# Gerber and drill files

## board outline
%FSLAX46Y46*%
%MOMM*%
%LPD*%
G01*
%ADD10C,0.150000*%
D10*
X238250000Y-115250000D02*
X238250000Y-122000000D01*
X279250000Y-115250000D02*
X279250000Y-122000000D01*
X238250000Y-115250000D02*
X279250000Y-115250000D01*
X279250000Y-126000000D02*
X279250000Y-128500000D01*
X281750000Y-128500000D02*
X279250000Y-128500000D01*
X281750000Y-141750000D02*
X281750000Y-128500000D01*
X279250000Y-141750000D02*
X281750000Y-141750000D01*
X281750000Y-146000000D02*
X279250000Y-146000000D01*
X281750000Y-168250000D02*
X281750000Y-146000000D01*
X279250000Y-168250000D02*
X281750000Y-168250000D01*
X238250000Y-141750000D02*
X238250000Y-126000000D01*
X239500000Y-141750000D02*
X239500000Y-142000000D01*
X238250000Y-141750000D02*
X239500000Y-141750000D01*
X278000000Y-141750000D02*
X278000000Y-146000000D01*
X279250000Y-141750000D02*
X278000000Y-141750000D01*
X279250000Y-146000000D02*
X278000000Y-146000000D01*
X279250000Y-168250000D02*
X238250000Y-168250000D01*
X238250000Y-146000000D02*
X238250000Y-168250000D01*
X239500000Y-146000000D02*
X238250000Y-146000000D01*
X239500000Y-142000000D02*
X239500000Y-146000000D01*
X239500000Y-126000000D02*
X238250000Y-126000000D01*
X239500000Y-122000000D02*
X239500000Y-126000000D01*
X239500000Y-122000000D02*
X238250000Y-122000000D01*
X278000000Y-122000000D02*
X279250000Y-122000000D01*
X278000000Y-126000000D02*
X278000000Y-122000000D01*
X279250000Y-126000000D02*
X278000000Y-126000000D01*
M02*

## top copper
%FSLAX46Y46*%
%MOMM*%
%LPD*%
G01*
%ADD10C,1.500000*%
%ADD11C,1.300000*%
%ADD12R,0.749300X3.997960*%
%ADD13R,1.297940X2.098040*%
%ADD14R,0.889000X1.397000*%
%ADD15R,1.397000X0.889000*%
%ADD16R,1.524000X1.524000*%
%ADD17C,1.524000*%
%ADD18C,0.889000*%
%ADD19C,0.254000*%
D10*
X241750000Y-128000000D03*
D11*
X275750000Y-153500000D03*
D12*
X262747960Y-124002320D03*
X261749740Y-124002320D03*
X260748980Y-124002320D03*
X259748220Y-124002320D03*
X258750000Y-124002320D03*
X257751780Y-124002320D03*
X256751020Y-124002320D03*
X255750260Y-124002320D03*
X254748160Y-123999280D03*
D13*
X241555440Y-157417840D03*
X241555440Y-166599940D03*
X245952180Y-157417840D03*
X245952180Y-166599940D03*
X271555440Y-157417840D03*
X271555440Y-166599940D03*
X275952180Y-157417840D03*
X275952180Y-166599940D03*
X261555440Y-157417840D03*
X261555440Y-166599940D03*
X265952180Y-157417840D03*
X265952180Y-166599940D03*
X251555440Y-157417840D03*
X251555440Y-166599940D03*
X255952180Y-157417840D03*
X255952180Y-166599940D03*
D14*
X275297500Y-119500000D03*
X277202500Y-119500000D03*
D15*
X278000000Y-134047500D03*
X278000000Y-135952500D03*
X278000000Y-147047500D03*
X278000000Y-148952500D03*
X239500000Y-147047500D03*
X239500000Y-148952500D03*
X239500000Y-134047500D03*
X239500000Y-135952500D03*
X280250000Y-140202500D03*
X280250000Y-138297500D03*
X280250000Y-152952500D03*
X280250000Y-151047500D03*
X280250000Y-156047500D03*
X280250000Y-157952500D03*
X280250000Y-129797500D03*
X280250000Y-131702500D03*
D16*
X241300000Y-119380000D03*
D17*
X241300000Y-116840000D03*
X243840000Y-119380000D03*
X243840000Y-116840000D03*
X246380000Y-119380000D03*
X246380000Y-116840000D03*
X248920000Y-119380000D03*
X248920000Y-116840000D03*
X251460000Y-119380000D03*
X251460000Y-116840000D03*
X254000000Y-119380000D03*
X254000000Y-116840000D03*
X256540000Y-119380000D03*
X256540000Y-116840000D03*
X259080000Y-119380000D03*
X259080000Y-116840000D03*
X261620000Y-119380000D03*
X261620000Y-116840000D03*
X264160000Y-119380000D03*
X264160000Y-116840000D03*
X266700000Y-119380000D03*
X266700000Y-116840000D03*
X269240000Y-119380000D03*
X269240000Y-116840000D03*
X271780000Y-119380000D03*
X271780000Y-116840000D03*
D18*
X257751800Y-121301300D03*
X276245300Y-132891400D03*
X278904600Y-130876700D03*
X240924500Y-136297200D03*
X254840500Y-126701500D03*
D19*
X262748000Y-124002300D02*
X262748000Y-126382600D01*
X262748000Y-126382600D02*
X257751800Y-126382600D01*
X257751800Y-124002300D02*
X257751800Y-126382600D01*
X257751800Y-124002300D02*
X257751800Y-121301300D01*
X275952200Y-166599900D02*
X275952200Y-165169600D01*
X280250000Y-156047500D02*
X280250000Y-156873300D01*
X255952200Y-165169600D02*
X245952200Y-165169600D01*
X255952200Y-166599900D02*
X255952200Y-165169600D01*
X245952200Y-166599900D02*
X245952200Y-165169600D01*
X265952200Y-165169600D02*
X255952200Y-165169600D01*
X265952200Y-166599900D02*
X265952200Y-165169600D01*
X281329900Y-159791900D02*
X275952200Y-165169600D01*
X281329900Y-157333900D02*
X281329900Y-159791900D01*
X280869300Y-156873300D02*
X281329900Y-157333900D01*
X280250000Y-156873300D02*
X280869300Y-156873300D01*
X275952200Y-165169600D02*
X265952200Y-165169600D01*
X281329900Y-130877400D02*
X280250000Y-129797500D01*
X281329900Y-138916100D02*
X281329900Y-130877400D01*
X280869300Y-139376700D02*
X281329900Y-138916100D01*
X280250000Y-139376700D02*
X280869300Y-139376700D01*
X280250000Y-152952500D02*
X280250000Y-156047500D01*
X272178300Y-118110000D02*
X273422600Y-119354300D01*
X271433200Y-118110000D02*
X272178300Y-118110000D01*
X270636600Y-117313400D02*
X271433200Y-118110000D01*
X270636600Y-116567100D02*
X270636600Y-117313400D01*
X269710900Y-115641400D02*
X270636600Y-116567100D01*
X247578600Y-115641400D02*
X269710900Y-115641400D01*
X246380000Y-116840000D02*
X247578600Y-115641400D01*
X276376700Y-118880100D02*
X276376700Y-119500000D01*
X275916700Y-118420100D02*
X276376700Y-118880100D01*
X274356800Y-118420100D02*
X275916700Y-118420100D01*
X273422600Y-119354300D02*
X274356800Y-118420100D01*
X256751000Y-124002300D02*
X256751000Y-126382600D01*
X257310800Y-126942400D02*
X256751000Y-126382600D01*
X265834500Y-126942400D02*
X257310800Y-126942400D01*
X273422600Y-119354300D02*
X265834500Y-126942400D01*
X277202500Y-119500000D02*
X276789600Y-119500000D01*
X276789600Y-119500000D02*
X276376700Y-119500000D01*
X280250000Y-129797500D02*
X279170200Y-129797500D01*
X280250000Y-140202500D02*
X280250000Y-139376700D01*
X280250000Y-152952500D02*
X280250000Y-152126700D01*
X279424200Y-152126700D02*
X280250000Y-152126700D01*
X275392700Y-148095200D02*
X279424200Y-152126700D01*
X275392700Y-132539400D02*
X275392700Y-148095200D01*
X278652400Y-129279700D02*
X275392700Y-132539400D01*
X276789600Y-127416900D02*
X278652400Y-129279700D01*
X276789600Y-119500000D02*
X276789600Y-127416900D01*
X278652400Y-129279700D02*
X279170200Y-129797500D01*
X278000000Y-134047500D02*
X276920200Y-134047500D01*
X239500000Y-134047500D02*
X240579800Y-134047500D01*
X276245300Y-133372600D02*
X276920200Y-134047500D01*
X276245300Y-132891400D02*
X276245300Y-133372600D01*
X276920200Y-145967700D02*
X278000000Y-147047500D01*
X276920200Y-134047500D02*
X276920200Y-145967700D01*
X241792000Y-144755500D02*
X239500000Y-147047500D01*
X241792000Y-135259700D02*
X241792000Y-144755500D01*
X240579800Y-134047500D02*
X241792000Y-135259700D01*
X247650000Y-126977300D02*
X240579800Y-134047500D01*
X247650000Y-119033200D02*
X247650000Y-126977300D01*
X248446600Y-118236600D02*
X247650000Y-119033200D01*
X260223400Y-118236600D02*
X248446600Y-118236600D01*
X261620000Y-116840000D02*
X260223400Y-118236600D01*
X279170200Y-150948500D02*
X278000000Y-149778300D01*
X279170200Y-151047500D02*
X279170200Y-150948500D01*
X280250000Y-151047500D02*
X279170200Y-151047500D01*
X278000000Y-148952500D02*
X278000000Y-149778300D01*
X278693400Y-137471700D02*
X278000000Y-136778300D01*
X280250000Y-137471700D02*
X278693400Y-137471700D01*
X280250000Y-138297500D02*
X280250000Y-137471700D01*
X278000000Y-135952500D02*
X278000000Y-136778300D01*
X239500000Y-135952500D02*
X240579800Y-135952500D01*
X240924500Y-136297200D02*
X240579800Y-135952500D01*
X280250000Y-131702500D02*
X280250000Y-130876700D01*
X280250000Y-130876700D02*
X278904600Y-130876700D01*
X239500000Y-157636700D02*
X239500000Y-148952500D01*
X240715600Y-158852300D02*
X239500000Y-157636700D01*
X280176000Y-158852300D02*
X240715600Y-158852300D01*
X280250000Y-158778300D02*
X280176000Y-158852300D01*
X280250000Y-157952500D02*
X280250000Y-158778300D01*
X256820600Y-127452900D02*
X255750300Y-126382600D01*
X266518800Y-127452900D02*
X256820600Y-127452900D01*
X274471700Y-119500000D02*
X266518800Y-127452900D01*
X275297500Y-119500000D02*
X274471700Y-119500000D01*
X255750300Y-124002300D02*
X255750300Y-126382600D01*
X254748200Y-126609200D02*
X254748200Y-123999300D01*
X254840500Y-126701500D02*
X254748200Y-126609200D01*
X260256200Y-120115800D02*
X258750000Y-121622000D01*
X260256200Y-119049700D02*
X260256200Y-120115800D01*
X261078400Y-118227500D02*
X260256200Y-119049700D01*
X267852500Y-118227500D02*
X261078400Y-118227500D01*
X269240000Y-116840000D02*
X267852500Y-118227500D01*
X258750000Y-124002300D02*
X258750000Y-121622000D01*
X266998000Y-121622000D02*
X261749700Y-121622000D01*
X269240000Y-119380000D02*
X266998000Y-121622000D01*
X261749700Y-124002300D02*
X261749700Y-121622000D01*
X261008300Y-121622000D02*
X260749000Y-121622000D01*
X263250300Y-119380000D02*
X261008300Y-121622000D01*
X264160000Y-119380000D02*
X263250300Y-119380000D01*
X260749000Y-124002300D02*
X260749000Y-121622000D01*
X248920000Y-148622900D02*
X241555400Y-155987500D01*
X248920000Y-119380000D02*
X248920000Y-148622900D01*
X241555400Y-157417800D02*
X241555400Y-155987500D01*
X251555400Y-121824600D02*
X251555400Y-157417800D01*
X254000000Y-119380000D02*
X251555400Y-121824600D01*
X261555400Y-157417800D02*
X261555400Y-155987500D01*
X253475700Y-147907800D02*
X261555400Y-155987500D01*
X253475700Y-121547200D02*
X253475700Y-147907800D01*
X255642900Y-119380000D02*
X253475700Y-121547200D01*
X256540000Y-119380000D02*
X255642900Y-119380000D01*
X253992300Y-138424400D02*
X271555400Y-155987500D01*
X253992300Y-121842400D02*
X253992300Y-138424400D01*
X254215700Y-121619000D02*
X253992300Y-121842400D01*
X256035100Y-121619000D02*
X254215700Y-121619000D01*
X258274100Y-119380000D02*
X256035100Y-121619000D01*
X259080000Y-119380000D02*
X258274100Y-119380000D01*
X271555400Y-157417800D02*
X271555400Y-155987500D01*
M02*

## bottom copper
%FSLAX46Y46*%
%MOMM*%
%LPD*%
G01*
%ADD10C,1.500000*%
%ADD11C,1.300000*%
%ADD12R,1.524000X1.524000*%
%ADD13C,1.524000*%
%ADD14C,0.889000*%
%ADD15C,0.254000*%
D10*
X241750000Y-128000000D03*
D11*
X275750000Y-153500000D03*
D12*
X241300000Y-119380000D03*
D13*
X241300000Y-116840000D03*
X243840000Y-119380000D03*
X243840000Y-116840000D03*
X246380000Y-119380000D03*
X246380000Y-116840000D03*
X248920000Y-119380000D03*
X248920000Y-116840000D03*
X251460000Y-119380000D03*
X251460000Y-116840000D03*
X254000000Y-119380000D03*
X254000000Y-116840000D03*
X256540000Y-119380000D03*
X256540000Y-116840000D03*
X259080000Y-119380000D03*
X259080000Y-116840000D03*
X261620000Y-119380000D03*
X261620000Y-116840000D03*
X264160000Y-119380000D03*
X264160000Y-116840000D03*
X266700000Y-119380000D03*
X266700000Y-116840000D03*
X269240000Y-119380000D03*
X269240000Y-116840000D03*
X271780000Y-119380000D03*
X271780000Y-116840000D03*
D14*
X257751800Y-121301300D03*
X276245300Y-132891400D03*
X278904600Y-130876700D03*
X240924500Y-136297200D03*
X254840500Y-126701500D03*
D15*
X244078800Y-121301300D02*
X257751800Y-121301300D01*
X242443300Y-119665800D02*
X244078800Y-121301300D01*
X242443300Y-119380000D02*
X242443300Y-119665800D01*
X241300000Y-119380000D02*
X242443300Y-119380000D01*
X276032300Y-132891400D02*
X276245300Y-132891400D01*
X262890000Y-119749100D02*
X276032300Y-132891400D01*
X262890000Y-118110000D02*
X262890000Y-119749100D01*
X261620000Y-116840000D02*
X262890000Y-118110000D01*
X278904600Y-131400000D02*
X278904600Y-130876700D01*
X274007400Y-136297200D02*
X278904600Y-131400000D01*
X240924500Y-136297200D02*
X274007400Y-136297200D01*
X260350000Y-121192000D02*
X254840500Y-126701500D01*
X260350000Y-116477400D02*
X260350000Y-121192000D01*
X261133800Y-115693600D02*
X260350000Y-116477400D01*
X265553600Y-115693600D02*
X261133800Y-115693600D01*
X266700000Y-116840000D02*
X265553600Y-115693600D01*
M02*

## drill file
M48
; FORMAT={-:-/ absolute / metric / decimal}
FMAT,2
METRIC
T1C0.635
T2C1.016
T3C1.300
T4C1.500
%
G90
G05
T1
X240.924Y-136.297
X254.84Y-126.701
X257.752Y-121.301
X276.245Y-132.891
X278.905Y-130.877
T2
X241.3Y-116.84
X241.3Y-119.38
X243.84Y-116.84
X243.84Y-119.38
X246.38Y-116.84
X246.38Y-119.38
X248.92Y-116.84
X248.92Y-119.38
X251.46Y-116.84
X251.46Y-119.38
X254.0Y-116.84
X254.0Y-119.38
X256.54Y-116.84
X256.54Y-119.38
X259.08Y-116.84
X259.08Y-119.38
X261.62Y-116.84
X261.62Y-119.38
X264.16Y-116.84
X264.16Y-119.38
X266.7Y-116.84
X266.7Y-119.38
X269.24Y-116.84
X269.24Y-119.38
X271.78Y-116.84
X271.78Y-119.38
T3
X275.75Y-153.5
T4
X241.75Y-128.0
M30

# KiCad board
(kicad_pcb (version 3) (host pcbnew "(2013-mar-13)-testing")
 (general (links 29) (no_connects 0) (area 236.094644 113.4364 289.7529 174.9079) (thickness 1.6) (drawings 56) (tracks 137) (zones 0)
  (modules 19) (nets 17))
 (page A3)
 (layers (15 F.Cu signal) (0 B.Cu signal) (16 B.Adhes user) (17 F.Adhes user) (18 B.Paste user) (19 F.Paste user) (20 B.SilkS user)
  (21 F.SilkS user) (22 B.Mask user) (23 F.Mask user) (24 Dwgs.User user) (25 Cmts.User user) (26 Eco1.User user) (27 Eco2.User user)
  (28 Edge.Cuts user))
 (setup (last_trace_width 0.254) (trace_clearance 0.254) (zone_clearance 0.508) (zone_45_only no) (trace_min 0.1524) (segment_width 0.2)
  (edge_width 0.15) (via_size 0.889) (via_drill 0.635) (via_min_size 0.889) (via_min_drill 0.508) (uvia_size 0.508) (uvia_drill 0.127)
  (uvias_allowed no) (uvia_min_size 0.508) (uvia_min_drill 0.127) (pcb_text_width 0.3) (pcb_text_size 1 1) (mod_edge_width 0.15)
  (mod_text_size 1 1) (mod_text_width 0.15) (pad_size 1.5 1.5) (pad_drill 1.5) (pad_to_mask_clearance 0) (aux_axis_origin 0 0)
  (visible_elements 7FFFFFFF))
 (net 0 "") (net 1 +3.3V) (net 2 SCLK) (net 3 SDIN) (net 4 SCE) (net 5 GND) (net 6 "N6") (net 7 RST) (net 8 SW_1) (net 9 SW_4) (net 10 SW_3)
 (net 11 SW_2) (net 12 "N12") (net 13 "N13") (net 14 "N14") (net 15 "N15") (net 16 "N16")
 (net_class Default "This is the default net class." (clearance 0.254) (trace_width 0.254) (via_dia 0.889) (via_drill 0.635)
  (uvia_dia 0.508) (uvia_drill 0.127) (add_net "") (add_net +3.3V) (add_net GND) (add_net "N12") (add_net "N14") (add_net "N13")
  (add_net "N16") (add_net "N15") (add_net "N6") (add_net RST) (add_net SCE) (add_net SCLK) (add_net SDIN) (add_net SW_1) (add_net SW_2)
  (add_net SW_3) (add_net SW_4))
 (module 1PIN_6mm (layer F.Cu) (at 241.75 128)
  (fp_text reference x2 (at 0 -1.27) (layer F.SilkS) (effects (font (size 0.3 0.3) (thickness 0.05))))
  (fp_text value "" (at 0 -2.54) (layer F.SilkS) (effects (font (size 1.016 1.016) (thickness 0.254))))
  (pad 1 thru_hole circle (at 0 0) (size 1.5 1.5) (drill 1.5) (layers *.Cu *.Mask F.SilkS)))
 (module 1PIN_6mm (layer F.Cu) (at 275.75 153.5)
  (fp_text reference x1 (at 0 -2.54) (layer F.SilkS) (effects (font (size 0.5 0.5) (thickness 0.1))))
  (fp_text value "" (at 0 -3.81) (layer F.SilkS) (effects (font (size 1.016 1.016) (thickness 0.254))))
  (pad 1 thru_hole circle (at 0 0) (size 1.3 1.3) (drill 1.3) (layers *.Cu *.Mask F.SilkS)))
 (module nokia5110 (layer F.Cu) (at 258.75 141)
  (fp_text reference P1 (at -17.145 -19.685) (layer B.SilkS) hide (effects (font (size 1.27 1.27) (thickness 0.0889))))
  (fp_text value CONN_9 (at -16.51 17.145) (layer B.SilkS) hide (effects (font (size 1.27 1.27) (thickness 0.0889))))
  (pad 9 smd rect (at 3.99796 -16.99768) (size 0.7493 3.99796) (layers F.Cu F.Paste F.Mask) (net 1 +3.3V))
  (pad 8 smd rect (at 2.99974 -16.99768) (size 0.7493 3.99796) (layers F.Cu F.Paste F.Mask) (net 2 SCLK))
  (pad 7 smd rect (at 1.99898 -16.99768) (size 0.7493 3.99796) (layers F.Cu F.Paste F.Mask) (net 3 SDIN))
  (pad 6 smd rect (at 0.99822 -16.99768) (size 0.7493 3.99796) (layers F.Cu F.Paste F.Mask))
  (pad 5 smd rect (at 0 -16.99768) (size 0.7493 3.99796) (layers F.Cu F.Paste F.Mask) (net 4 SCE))
  (pad 4 smd rect (at -0.99822 -16.99768) (size 0.7493 3.99796) (layers F.Cu F.Paste F.Mask) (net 1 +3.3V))
  (pad 3 smd rect (at -1.99898 -16.99768) (size 0.7493 3.99796) (layers F.Cu F.Paste F.Mask) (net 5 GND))
  (pad 2 smd rect (at -2.99974 -16.99768) (size 0.7493 3.99796) (layers F.Cu F.Paste F.Mask) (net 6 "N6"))
  (pad 1 smd rect (at -4.00184 -17.00072) (size 0.7493 3.99796) (layers F.Cu F.Paste F.Mask) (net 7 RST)))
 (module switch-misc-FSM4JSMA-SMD (layer F.Cu) (at 243.75 162)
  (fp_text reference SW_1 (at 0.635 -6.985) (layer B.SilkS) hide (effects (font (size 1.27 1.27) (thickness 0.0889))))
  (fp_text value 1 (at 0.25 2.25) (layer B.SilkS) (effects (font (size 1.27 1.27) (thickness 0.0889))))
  (pad P$1 smd rect (at -2.19456 -4.58216) (size 1.29794 2.09804) (layers F.Cu F.Paste F.Mask) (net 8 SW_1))
  (pad P$2 smd rect (at -2.19456 4.59994) (size 1.29794 2.09804) (layers F.Cu F.Paste F.Mask))
  (pad P$3 smd rect (at 2.20218 -4.58216) (size 1.29794 2.09804) (layers F.Cu F.Paste F.Mask))
  (pad P$4 smd rect (at 2.20218 4.59994) (size 1.29794 2.09804) (layers F.Cu F.Paste F.Mask) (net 5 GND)))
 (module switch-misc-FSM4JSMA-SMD (layer F.Cu) (at 273.75 162)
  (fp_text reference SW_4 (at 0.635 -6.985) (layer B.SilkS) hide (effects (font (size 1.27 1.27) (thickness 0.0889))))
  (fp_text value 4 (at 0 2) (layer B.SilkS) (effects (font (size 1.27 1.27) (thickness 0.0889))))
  (pad P$1 smd rect (at -2.19456 -4.58216) (size 1.29794 2.09804) (layers F.Cu F.Paste F.Mask) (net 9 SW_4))
  (pad P$2 smd rect (at -2.19456 4.59994) (size 1.29794 2.09804) (layers F.Cu F.Paste F.Mask))
  (pad P$3 smd rect (at 2.20218 -4.58216) (size 1.29794 2.09804) (layers F.Cu F.Paste F.Mask))
  (pad P$4 smd rect (at 2.20218 4.59994) (size 1.29794 2.09804) (layers F.Cu F.Paste F.Mask) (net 5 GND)))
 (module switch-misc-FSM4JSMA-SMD (layer F.Cu) (at 263.75 162)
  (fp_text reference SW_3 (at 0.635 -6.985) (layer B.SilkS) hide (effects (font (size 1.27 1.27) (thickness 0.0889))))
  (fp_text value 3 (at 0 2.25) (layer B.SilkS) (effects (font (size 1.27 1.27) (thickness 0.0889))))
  (pad P$1 smd rect (at -2.19456 -4.58216) (size 1.29794 2.09804) (layers F.Cu F.Paste F.Mask) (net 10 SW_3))
  (pad P$2 smd rect (at -2.19456 4.59994) (size 1.29794 2.09804) (layers F.Cu F.Paste F.Mask))
  (pad P$3 smd rect (at 2.20218 -4.58216) (size 1.29794 2.09804) (layers F.Cu F.Paste F.Mask))
  (pad P$4 smd rect (at 2.20218 4.59994) (size 1.29794 2.09804) (layers F.Cu F.Paste F.Mask) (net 5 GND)))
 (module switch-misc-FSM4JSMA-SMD (layer F.Cu) (at 253.75 162)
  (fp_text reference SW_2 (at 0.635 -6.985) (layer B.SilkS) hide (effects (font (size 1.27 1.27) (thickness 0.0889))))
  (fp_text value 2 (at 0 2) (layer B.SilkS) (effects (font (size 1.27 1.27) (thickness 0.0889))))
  (pad P$1 smd rect (at -2.19456 -4.58216) (size 1.29794 2.09804) (layers F.Cu F.Paste F.Mask) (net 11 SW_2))
  (pad P$2 smd rect (at -2.19456 4.59994) (size 1.29794 2.09804) (layers F.Cu F.Paste F.Mask))
  (pad P$3 smd rect (at 2.20218 -4.58216) (size 1.29794 2.09804) (layers F.Cu F.Paste F.Mask))
  (pad P$4 smd rect (at 2.20218 4.59994) (size 1.29794 2.09804) (layers F.Cu F.Paste F.Mask) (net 5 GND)))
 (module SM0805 (layer F.Cu) (at 276.25 119.5)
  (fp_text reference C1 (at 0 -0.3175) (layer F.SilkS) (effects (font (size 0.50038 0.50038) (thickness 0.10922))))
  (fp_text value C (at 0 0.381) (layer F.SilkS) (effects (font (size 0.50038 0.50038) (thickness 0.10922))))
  (pad 1 smd rect (at -0.9525 0) (size 0.889 1.397) (layers F.Cu F.Paste F.Mask) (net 6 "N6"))
  (pad 2 smd rect (at 0.9525 0) (size 0.889 1.397) (layers F.Cu F.Paste F.Mask) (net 5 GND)))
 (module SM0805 (layer F.Cu) (at 278 135 270)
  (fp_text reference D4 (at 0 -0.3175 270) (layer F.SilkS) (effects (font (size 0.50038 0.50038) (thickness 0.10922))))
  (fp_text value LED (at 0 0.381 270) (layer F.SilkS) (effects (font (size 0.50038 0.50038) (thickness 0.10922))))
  (pad 1 smd rect (at -0.9525 0 270) (size 0.889 1.397) (layers F.Cu F.Paste F.Mask) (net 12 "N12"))
  (pad 2 smd rect (at 0.9525 0 270) (size 0.889 1.397) (layers F.Cu F.Paste F.Mask) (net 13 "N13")))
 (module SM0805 (layer F.Cu) (at 278 148 270)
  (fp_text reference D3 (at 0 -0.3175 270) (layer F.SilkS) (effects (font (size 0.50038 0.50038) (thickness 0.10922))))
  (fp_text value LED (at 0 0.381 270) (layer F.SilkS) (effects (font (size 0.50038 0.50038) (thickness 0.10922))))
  (pad 1 smd rect (at -0.9525 0 270) (size 0.889 1.397) (layers F.Cu F.Paste F.Mask) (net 12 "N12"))
  (pad 2 smd rect (at 0.9525 0 270) (size 0.889 1.397) (layers F.Cu F.Paste F.Mask) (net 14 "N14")))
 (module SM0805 (layer F.Cu) (at 239.5 148 270)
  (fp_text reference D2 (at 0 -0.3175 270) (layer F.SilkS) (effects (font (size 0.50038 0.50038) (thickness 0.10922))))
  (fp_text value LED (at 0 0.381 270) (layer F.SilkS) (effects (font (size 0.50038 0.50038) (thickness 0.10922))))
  (pad 1 smd rect (at -0.9525 0 270) (size 0.889 1.397) (layers F.Cu F.Paste F.Mask) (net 12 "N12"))
  (pad 2 smd rect (at 0.9525 0 270) (size 0.889 1.397) (layers F.Cu F.Paste F.Mask) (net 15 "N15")))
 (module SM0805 (layer F.Cu) (at 239.5 135 270)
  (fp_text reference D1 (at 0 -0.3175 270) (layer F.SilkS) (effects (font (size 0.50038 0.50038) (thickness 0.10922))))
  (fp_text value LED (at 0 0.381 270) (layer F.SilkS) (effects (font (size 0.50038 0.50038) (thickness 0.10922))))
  (pad 1 smd rect (at -0.9525 0 270) (size 0.889 1.397) (layers F.Cu F.Paste F.Mask) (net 12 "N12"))
  (pad 2 smd rect (at 0.9525 0 270) (size 0.889 1.397) (layers F.Cu F.Paste F.Mask) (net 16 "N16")))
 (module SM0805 (layer F.Cu) (at 280.25 139.25 90)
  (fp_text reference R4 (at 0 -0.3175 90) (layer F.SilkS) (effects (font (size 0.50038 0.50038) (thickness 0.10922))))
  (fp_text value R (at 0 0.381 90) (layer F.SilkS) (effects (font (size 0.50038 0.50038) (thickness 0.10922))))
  (pad 1 smd rect (at -0.9525 0 90) (size 0.889 1.397) (layers F.Cu F.Paste F.Mask) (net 5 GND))
  (pad 2 smd rect (at 0.9525 0 90) (size 0.889 1.397) (layers F.Cu F.Paste F.Mask) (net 13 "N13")))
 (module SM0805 (layer F.Cu) (at 280.25 152 90)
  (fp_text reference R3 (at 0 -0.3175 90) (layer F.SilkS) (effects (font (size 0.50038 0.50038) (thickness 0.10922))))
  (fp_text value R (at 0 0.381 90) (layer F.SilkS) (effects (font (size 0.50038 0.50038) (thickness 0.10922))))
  (pad 1 smd rect (at -0.9525 0 90) (size 0.889 1.397) (layers F.Cu F.Paste F.Mask) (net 5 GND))
  (pad 2 smd rect (at 0.9525 0 90) (size 0.889 1.397) (layers F.Cu F.Paste F.Mask) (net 14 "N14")))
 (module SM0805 (layer F.Cu) (at 280.25 157 270)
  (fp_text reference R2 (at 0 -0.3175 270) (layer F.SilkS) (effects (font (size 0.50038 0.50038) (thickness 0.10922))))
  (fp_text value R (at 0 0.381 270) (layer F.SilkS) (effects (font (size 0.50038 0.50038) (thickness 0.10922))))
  (pad 1 smd rect (at -0.9525 0 270) (size 0.889 1.397) (layers F.Cu F.Paste F.Mask) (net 5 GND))
  (pad 2 smd rect (at 0.9525 0 270) (size 0.889 1.397) (layers F.Cu F.Paste F.Mask) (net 15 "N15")))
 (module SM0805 (layer F.Cu) (at 280.25 130.75 270)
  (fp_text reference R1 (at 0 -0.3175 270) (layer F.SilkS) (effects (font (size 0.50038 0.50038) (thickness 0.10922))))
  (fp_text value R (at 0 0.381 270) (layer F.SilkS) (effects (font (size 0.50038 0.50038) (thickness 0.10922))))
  (pad 1 smd rect (at -0.9525 0 270) (size 0.889 1.397) (layers F.Cu F.Paste F.Mask) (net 5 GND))
  (pad 2 smd rect (at 0.9525 0 270) (size 0.889 1.397) (layers F.Cu F.Paste F.Mask) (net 16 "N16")))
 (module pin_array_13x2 (layer F.Cu) (at 256.54 118.11)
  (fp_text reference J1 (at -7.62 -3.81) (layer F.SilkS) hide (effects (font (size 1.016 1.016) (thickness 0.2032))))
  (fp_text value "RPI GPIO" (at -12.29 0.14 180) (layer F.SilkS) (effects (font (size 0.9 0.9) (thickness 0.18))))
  (pad 1 thru_hole rect (at -15.24 1.27) (size 1.524 1.524) (drill 1.016) (layers *.Cu *.Mask F.SilkS) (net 1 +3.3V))
  (pad 2 thru_hole circle (at -15.24 -1.27) (size 1.524 1.524) (drill 1.016) (layers *.Cu *.Mask F.SilkS))
  (pad 3 thru_hole circle (at -12.7 1.27) (size 1.524 1.524) (drill 1.016) (layers *.Cu *.Mask F.SilkS))
  (pad 4 thru_hole circle (at -12.7 -1.27) (size 1.524 1.524) (drill 1.016) (layers *.Cu *.Mask F.SilkS))
  (pad 5 thru_hole circle (at -10.16 1.27) (size 1.524 1.524) (drill 1.016) (layers *.Cu *.Mask F.SilkS))
  (pad 6 thru_hole circle (at -10.16 -1.27) (size 1.524 1.524) (drill 1.016) (layers *.Cu *.Mask F.SilkS) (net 5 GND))
  (pad 7 thru_hole circle (at -7.62 1.27) (size 1.524 1.524) (drill 1.016) (layers *.Cu *.Mask F.SilkS) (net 8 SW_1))
  (pad 8 thru_hole circle (at -7.62 -1.27) (size 1.524 1.524) (drill 1.016) (layers *.Cu *.Mask F.SilkS))
  (pad 9 thru_hole circle (at -5.08 1.27) (size 1.524 1.524) (drill 1.016) (layers *.Cu *.Mask F.SilkS))
  (pad 10 thru_hole circle (at -5.08 -1.27) (size 1.524 1.524) (drill 1.016) (layers *.Cu *.Mask F.SilkS))
  (pad 11 thru_hole circle (at -2.54 1.27) (size 1.524 1.524) (drill 1.016) (layers *.Cu *.Mask F.SilkS) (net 11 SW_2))
  (pad 12 thru_hole circle (at -2.54 -1.27) (size 1.524 1.524) (drill 1.016) (layers *.Cu *.Mask F.SilkS))
  (pad 13 thru_hole circle (at 0 1.27) (size 1.524 1.524) (drill 1.016) (layers *.Cu *.Mask F.SilkS) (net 10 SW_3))
  (pad 14 thru_hole circle (at 0 -1.27) (size 1.524 1.524) (drill 1.016) (layers *.Cu *.Mask F.SilkS))
  (pad 15 thru_hole circle (at 2.54 1.27) (size 1.524 1.524) (drill 1.016) (layers *.Cu *.Mask F.SilkS) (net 9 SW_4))
  (pad 16 thru_hole circle (at 2.54 -1.27) (size 1.524 1.524) (drill 1.016) (layers *.Cu *.Mask F.SilkS))
  (pad 17 thru_hole circle (at 5.08 1.27) (size 1.524 1.524) (drill 1.016) (layers *.Cu *.Mask F.SilkS))
  (pad 18 thru_hole circle (at 5.08 -1.27) (size 1.524 1.524) (drill 1.016) (layers *.Cu *.Mask F.SilkS) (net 12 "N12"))
  (pad 19 thru_hole circle (at 7.62 1.27) (size 1.524 1.524) (drill 1.016) (layers *.Cu *.Mask F.SilkS) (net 3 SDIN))
  (pad 20 thru_hole circle (at 7.62 -1.27) (size 1.524 1.524) (drill 1.016) (layers *.Cu *.Mask F.SilkS))
  (pad 21 thru_hole circle (at 10.16 1.27) (size 1.524 1.524) (drill 1.016) (layers *.Cu *.Mask F.SilkS))
  (pad 22 thru_hole circle (at 10.16 -1.27) (size 1.524 1.524) (drill 1.016) (layers *.Cu *.Mask F.SilkS) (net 7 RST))
  (pad 23 thru_hole circle (at 12.7 1.27) (size 1.524 1.524) (drill 1.016) (layers *.Cu *.Mask F.SilkS) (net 2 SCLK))
  (pad 24 thru_hole circle (at 12.7 -1.27) (size 1.524 1.524) (drill 1.016) (layers *.Cu *.Mask F.SilkS) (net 4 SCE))
  (pad 25 thru_hole circle (at 15.24 1.27) (size 1.524 1.524) (drill 1.016) (layers *.Cu *.Mask F.SilkS))
  (pad 26 thru_hole circle (at 15.24 -1.27) (size 1.524 1.524) (drill 1.016) (layers *.Cu *.Mask F.SilkS)))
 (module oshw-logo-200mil (layer F.Cu) (at 279.25 165.5)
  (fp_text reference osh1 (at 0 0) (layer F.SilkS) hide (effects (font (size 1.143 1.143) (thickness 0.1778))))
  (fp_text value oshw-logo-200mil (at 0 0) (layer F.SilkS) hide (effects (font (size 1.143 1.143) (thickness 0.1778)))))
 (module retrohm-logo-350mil (layer F.Cu) (at 239.5 162.5 90)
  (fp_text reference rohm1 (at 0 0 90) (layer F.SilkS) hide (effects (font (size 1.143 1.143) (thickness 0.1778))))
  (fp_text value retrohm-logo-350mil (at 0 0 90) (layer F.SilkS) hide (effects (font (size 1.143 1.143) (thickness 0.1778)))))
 (gr_line (start 238.25 115.25) (end 238.25 122) (angle 90) (layer Edge.Cuts) (width 0.15))
 (gr_line (start 279.25 115.25) (end 279.25 122) (angle 90) (layer Edge.Cuts) (width 0.15))
 (gr_line (start 238.25 115.25) (end 279.25 115.25) (angle 90) (layer Edge.Cuts) (width 0.15))
 (gr_line (start 279.25 126) (end 279.25 128.5) (angle 90) (layer Edge.Cuts) (width 0.15))
 (gr_line (start 281.75 128.5) (end 279.25 128.5) (angle 90) (layer Edge.Cuts) (width 0.15))
 (gr_line (start 281.75 141.75) (end 281.75 128.5) (angle 90) (layer Edge.Cuts) (width 0.15))
 (gr_line (start 279.25 141.75) (end 281.75 141.75) (angle 90) (layer Edge.Cuts) (width 0.15))
 (gr_line (start 281.75 146) (end 279.25 146) (angle 90) (layer Edge.Cuts) (width 0.15))
 (gr_line (start 281.75 168.25) (end 281.75 146) (angle 90) (layer Edge.Cuts) (width 0.15))
 (gr_line (start 279.25 168.25) (end 281.75 168.25) (angle 90) (layer Edge.Cuts) (width 0.15))
 (gr_line (start 238.25 141.75) (end 238.25 126) (angle 90) (layer Edge.Cuts) (width 0.15))
 (gr_line (start 239.5 141.75) (end 239.5 142) (angle 90) (layer Edge.Cuts) (width 0.15))
 (gr_line (start 238.25 141.75) (end 239.5 141.75) (angle 90) (layer Edge.Cuts) (width 0.15))
 (gr_line (start 278 141.75) (end 278 146) (angle 90) (layer Edge.Cuts) (width 0.15))
 (gr_line (start 279.25 141.75) (end 278 141.75) (angle 90) (layer Edge.Cuts) (width 0.15))
 (gr_line (start 279.25 146) (end 278 146) (angle 90) (layer Edge.Cuts) (width 0.15))
 (gr_line (start 279.25 168.25) (end 238.25 168.25) (angle 90) (layer Edge.Cuts) (width 0.15))
 (gr_line (start 238.25 146) (end 238.25 168.25) (angle 90) (layer Edge.Cuts) (width 0.15))
 (gr_line (start 239.5 146) (end 238.25 146) (angle 90) (layer Edge.Cuts) (width 0.15))
 (gr_line (start 239.5 142) (end 239.5 146) (angle 90) (layer Edge.Cuts) (width 0.15))
 (gr_line (start 239.5 126) (end 238.25 126) (angle 90) (layer Edge.Cuts) (width 0.15))
 (gr_line (start 239.5 122) (end 239.5 126) (angle 90) (layer Edge.Cuts) (width 0.15))
 (gr_line (start 239.5 122) (end 238.25 122) (angle 90) (layer Edge.Cuts) (width 0.15))
 (gr_line (start 278 122) (end 279.25 122) (angle 90) (layer Edge.Cuts) (width 0.15))
 (gr_line (start 278 126) (end 278 122) (angle 90) (layer Edge.Cuts) (width 0.15))
 (gr_line (start 279.25 126) (end 278 126) (angle 90) (layer Edge.Cuts) (width 0.15))
 (via (at 257.7518 121.3013) (size 0.889) (layers F.Cu B.Cu) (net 1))
 (segment (start 262.748 124.0023) (end 262.748 126.3826) (width 0.254) (layer F.Cu) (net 1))
 (segment (start 262.748 126.3826) (end 257.7518 126.3826) (width 0.254) (layer F.Cu) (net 1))
 (segment (start 257.7518 124.0023) (end 257.7518 126.3826) (width 0.254) (layer F.Cu) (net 1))
 (segment (start 244.0788 121.3013) (end 257.7518 121.3013) (width 0.254) (layer B.Cu) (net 1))
 (segment (start 242.4433 119.6658) (end 244.0788 121.3013) (width 0.254) (layer B.Cu) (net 1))
 (segment (start 242.4433 119.38) (end 242.4433 119.6658) (width 0.254) (layer B.Cu) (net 1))
 (segment (start 257.7518 124.0023) (end 257.7518 121.3013) (width 0.254) (layer F.Cu) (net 1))
 (segment (start 241.3 119.38) (end 242.4433 119.38) (width 0.254) (layer B.Cu) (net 1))
 (segment (start 275.9522 166.5999) (end 275.9522 165.1696) (width 0.254) (layer F.Cu) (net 5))
 (segment (start 280.25 156.0475) (end 280.25 156.8733) (width 0.254) (layer F.Cu) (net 5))
 (segment (start 255.9522 165.1696) (end 245.9522 165.1696) (width 0.254) (layer F.Cu) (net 5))
 (segment (start 255.9522 166.5999) (end 255.9522 165.1696) (width 0.254) (layer F.Cu) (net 5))
 (segment (start 245.9522 166.5999) (end 245.9522 165.1696) (width 0.254) (layer F.Cu) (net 5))
 (segment (start 265.9522 165.1696) (end 255.9522 165.1696) (width 0.254) (layer F.Cu) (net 5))
 (segment (start 265.9522 166.5999) (end 265.9522 165.1696) (width 0.254) (layer F.Cu) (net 5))
 (segment (start 281.3299 159.7919) (end 275.9522 165.1696) (width 0.254) (layer F.Cu) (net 5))
 (segment (start 281.3299 157.3339) (end 281.3299 159.7919) (width 0.254) (layer F.Cu) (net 5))
 (segment (start 280.8693 156.8733) (end 281.3299 157.3339) (width 0.254) (layer F.Cu) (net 5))
 (segment (start 280.25 156.8733) (end 280.8693 156.8733) (width 0.254) (layer F.Cu) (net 5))
 (segment (start 275.9522 165.1696) (end 265.9522 165.1696) (width 0.254) (layer F.Cu) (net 5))
 (segment (start 281.3299 130.8774) (end 280.25 129.7975) (width 0.254) (layer F.Cu) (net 5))
 (segment (start 281.3299 138.9161) (end 281.3299 130.8774) (width 0.254) (layer F.Cu) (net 5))
 (segment (start 280.8693 139.3767) (end 281.3299 138.9161) (width 0.254) (layer F.Cu) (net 5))
 (segment (start 280.25 139.3767) (end 280.8693 139.3767) (width 0.254) (layer F.Cu) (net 5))
 (segment (start 280.25 152.9525) (end 280.25 156.0475) (width 0.254) (layer F.Cu) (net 5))
 (segment (start 272.1783 118.11) (end 273.4226 119.3543) (width 0.254) (layer F.Cu) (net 5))
 (segment (start 271.4332 118.11) (end 272.1783 118.11) (width 0.254) (layer F.Cu) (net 5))
 (segment (start 270.6366 117.3134) (end 271.4332 118.11) (width 0.254) (layer F.Cu) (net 5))
 (segment (start 270.6366 116.5671) (end 270.6366 117.3134) (width 0.254) (layer F.Cu) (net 5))
 (segment (start 269.7109 115.6414) (end 270.6366 116.5671) (width 0.254) (layer F.Cu) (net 5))
 (segment (start 247.5786 115.6414) (end 269.7109 115.6414) (width 0.254) (layer F.Cu) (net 5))
 (segment (start 246.38 116.84) (end 247.5786 115.6414) (width 0.254) (layer F.Cu) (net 5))
 (segment (start 276.3767 118.8801) (end 276.3767 119.5) (width 0.254) (layer F.Cu) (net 5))
 (segment (start 275.9167 118.4201) (end 276.3767 118.8801) (width 0.254) (layer F.Cu) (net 5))
 (segment (start 274.3568 118.4201) (end 275.9167 118.4201) (width 0.254) (layer F.Cu) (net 5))
 (segment (start 273.4226 119.3543) (end 274.3568 118.4201) (width 0.254) (layer F.Cu) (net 5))
 (segment (start 256.751 124.0023) (end 256.751 126.3826) (width 0.254) (layer F.Cu) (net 5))
 (segment (start 257.3108 126.9424) (end 256.751 126.3826) (width 0.254) (layer F.Cu) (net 5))
 (segment (start 265.8345 126.9424) (end 257.3108 126.9424) (width 0.254) (layer F.Cu) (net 5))
 (segment (start 273.4226 119.3543) (end 265.8345 126.9424) (width 0.254) (layer F.Cu) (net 5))
 (segment (start 277.2025 119.5) (end 276.7896 119.5) (width 0.254) (layer F.Cu) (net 5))
 (segment (start 276.7896 119.5) (end 276.3767 119.5) (width 0.254) (layer F.Cu) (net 5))
 (segment (start 280.25 129.7975) (end 279.1702 129.7975) (width 0.254) (layer F.Cu) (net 5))
 (segment (start 280.25 140.2025) (end 280.25 139.3767) (width 0.254) (layer F.Cu) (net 5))
 (segment (start 280.25 152.9525) (end 280.25 152.1267) (width 0.254) (layer F.Cu) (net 5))
 (segment (start 279.4242 152.1267) (end 280.25 152.1267) (width 0.254) (layer F.Cu) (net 5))
 (segment (start 275.3927 148.0952) (end 279.4242 152.1267) (width 0.254) (layer F.Cu) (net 5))
 (segment (start 275.3927 132.5394) (end 275.3927 148.0952) (width 0.254) (layer F.Cu) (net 5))
 (segment (start 278.6524 129.2797) (end 275.3927 132.5394) (width 0.254) (layer F.Cu) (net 5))
 (segment (start 276.7896 127.4169) (end 278.6524 129.2797) (width 0.254) (layer F.Cu) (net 5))
 (segment (start 276.7896 119.5) (end 276.7896 127.4169) (width 0.254) (layer F.Cu) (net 5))
 (segment (start 278.6524 129.2797) (end 279.1702 129.7975) (width 0.254) (layer F.Cu) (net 5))
 (via (at 276.2453 132.8914) (size 0.889) (layers F.Cu B.Cu) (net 12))
 (segment (start 278 134.0475) (end 276.9202 134.0475) (width 0.254) (layer F.Cu) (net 12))
 (segment (start 276.0323 132.8914) (end 276.2453 132.8914) (width 0.254) (layer B.Cu) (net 12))
 (segment (start 262.89 119.7491) (end 276.0323 132.8914) (width 0.254) (layer B.Cu) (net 12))
 (segment (start 262.89 118.11) (end 262.89 119.7491) (width 0.254) (layer B.Cu) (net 12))
 (segment (start 261.62 116.84) (end 262.89 118.11) (width 0.254) (layer B.Cu) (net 12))
 (segment (start 239.5 134.0475) (end 240.5798 134.0475) (width 0.254) (layer F.Cu) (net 12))
 (segment (start 276.2453 133.3726) (end 276.9202 134.0475) (width 0.254) (layer F.Cu) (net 12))
 (segment (start 276.2453 132.8914) (end 276.2453 133.3726) (width 0.254) (layer F.Cu) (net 12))
 (segment (start 276.9202 145.9677) (end 278 147.0475) (width 0.254) (layer F.Cu) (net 12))
 (segment (start 276.9202 134.0475) (end 276.9202 145.9677) (width 0.254) (layer F.Cu) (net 12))
 (segment (start 241.792 144.7555) (end 239.5 147.0475) (width 0.254) (layer F.Cu) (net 12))
 (segment (start 241.792 135.2597) (end 241.792 144.7555) (width 0.254) (layer F.Cu) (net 12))
 (segment (start 240.5798 134.0475) (end 241.792 135.2597) (width 0.254) (layer F.Cu) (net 12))
 (segment (start 247.65 126.9773) (end 240.5798 134.0475) (width 0.254) (layer F.Cu) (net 12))
 (segment (start 247.65 119.0332) (end 247.65 126.9773) (width 0.254) (layer F.Cu) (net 12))
 (segment (start 248.4466 118.2366) (end 247.65 119.0332) (width 0.254) (layer F.Cu) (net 12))
 (segment (start 260.2234 118.2366) (end 248.4466 118.2366) (width 0.254) (layer F.Cu) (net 12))
 (segment (start 261.62 116.84) (end 260.2234 118.2366) (width 0.254) (layer F.Cu) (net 12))
 (segment (start 279.1702 150.9485) (end 278 149.7783) (width 0.254) (layer F.Cu) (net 14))
 (segment (start 279.1702 151.0475) (end 279.1702 150.9485) (width 0.254) (layer F.Cu) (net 14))
 (segment (start 280.25 151.0475) (end 279.1702 151.0475) (width 0.254) (layer F.Cu) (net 14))
 (segment (start 278 148.9525) (end 278 149.7783) (width 0.254) (layer F.Cu) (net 14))
 (segment (start 278.6934 137.4717) (end 278 136.7783) (width 0.254) (layer F.Cu) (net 13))
 (segment (start 280.25 137.4717) (end 278.6934 137.4717) (width 0.254) (layer F.Cu) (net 13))
 (segment (start 280.25 138.2975) (end 280.25 137.4717) (width 0.254) (layer F.Cu) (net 13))
 (segment (start 278 135.9525) (end 278 136.7783) (width 0.254) (layer F.Cu) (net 13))
 (via (at 278.9046 130.8767) (size 0.889) (layers F.Cu B.Cu) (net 16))
 (via (at 240.9245 136.2972) (size 0.889) (layers F.Cu B.Cu) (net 16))
 (segment (start 239.5 135.9525) (end 240.5798 135.9525) (width 0.254) (layer F.Cu) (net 16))
 (segment (start 240.9245 136.2972) (end 240.5798 135.9525) (width 0.254) (layer F.Cu) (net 16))
 (segment (start 280.25 131.7025) (end 280.25 130.8767) (width 0.254) (layer F.Cu) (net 16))
 (segment (start 280.25 130.8767) (end 278.9046 130.8767) (width 0.254) (layer F.Cu) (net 16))
 (segment (start 278.9046 131.4) (end 278.9046 130.8767) (width 0.254) (layer B.Cu) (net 16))
 (segment (start 274.0074 136.2972) (end 278.9046 131.4) (width 0.254) (layer B.Cu) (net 16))
 (segment (start 240.9245 136.2972) (end 274.0074 136.2972) (width 0.254) (layer B.Cu) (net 16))
 (segment (start 239.5 157.6367) (end 239.5 148.9525) (width 0.254) (layer F.Cu) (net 15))
 (segment (start 240.7156 158.8523) (end 239.5 157.6367) (width 0.254) (layer F.Cu) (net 15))
 (segment (start 280.176 158.8523) (end 240.7156 158.8523) (width 0.254) (layer F.Cu) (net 15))
 (segment (start 280.25 158.7783) (end 280.176 158.8523) (width 0.254) (layer F.Cu) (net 15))
 (segment (start 280.25 157.9525) (end 280.25 158.7783) (width 0.254) (layer F.Cu) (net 15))
 (segment (start 256.8206 127.4529) (end 255.7503 126.3826) (width 0.254) (layer F.Cu) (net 6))
 (segment (start 266.5188 127.4529) (end 256.8206 127.4529) (width 0.254) (layer F.Cu) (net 6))
 (segment (start 274.4717 119.5) (end 266.5188 127.4529) (width 0.254) (layer F.Cu) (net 6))
 (segment (start 275.2975 119.5) (end 274.4717 119.5) (width 0.254) (layer F.Cu) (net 6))
 (segment (start 255.7503 124.0023) (end 255.7503 126.3826) (width 0.254) (layer F.Cu) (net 6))
 (via (at 254.8405 126.7015) (size 0.889) (layers F.Cu B.Cu) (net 7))
 (segment (start 260.35 121.192) (end 254.8405 126.7015) (width 0.254) (layer B.Cu) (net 7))
 (segment (start 260.35 116.4774) (end 260.35 121.192) (width 0.254) (layer B.Cu) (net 7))
 (segment (start 261.1338 115.6936) (end 260.35 116.4774) (width 0.254) (layer B.Cu) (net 7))
 (segment (start 265.5536 115.6936) (end 261.1338 115.6936) (width 0.254) (layer B.Cu) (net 7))
 (segment (start 266.7 116.84) (end 265.5536 115.6936) (width 0.254) (layer B.Cu) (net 7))
 (segment (start 254.7482 126.6092) (end 254.7482 123.9993) (width 0.254) (layer F.Cu) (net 7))
 (segment (start 254.8405 126.7015) (end 254.7482 126.6092) (width 0.254) (layer F.Cu) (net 7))
 (segment (start 260.2562 120.1158) (end 258.75 121.622) (width 0.254) (layer F.Cu) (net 4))
 (segment (start 260.2562 119.0497) (end 260.2562 120.1158) (width 0.254) (layer F.Cu) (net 4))
 (segment (start 261.0784 118.2275) (end 260.2562 119.0497) (width 0.254) (layer F.Cu) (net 4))
 (segment (start 267.8525 118.2275) (end 261.0784 118.2275) (width 0.254) (layer F.Cu) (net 4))
 (segment (start 269.24 116.84) (end 267.8525 118.2275) (width 0.254) (layer F.Cu) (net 4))
 (segment (start 258.75 124.0023) (end 258.75 121.622) (width 0.254) (layer F.Cu) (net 4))
 (segment (start 266.998 121.622) (end 261.7497 121.622) (width 0.254) (layer F.Cu) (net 2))
 (segment (start 269.24 119.38) (end 266.998 121.622) (width 0.254) (layer F.Cu) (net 2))
 (segment (start 261.7497 124.0023) (end 261.7497 121.622) (width 0.254) (layer F.Cu) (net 2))
 (segment (start 261.0083 121.622) (end 260.749 121.622) (width 0.254) (layer F.Cu) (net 3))
 (segment (start 263.2503 119.38) (end 261.0083 121.622) (width 0.254) (layer F.Cu) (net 3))
 (segment (start 264.16 119.38) (end 263.2503 119.38) (width 0.254) (layer F.Cu) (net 3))
 (segment (start 260.749 124.0023) (end 260.749 121.622) (width 0.254) (layer F.Cu) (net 3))
 (segment (start 248.92 148.6229) (end 241.5554 155.9875) (width 0.254) (layer F.Cu) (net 8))
 (segment (start 248.92 119.38) (end 248.92 148.6229) (width 0.254) (layer F.Cu) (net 8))
 (segment (start 241.5554 157.4178) (end 241.5554 155.9875) (width 0.254) (layer F.Cu) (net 8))
 (segment (start 251.5554 121.8246) (end 251.5554 157.4178) (width 0.254) (layer F.Cu) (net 11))
 (segment (start 254 119.38) (end 251.5554 121.8246) (width 0.254) (layer F.Cu) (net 11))
 (segment (start 261.5554 157.4178) (end 261.5554 155.9875) (width 0.254) (layer F.Cu) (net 10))
 (segment (start 253.4757 147.9078) (end 261.5554 155.9875) (width 0.254) (layer F.Cu) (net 10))
 (segment (start 253.4757 121.5472) (end 253.4757 147.9078) (width 0.254) (layer F.Cu) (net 10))
 (segment (start 255.6429 119.38) (end 253.4757 121.5472) (width 0.254) (layer F.Cu) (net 10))
 (segment (start 256.54 119.38) (end 255.6429 119.38) (width 0.254) (layer F.Cu) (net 10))
 (segment (start 253.9923 138.4244) (end 271.5554 155.9875) (width 0.254) (layer F.Cu) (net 9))
 (segment (start 253.9923 121.8424) (end 253.9923 138.4244) (width 0.254) (layer F.Cu) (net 9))
 (segment (start 254.2157 121.619) (end 253.9923 121.8424) (width 0.254) (layer F.Cu) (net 9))
 (segment (start 256.0351 121.619) (end 254.2157 121.619) (width 0.254) (layer F.Cu) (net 9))
 (segment (start 258.2741 119.38) (end 256.0351 121.619) (width 0.254) (layer F.Cu) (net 9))
 (segment (start 259.08 119.38) (end 258.2741 119.38) (width 0.254) (layer F.Cu) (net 9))
 (segment (start 271.5554 157.4178) (end 271.5554 155.9875) (width 0.254) (layer F.Cu) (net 9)))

